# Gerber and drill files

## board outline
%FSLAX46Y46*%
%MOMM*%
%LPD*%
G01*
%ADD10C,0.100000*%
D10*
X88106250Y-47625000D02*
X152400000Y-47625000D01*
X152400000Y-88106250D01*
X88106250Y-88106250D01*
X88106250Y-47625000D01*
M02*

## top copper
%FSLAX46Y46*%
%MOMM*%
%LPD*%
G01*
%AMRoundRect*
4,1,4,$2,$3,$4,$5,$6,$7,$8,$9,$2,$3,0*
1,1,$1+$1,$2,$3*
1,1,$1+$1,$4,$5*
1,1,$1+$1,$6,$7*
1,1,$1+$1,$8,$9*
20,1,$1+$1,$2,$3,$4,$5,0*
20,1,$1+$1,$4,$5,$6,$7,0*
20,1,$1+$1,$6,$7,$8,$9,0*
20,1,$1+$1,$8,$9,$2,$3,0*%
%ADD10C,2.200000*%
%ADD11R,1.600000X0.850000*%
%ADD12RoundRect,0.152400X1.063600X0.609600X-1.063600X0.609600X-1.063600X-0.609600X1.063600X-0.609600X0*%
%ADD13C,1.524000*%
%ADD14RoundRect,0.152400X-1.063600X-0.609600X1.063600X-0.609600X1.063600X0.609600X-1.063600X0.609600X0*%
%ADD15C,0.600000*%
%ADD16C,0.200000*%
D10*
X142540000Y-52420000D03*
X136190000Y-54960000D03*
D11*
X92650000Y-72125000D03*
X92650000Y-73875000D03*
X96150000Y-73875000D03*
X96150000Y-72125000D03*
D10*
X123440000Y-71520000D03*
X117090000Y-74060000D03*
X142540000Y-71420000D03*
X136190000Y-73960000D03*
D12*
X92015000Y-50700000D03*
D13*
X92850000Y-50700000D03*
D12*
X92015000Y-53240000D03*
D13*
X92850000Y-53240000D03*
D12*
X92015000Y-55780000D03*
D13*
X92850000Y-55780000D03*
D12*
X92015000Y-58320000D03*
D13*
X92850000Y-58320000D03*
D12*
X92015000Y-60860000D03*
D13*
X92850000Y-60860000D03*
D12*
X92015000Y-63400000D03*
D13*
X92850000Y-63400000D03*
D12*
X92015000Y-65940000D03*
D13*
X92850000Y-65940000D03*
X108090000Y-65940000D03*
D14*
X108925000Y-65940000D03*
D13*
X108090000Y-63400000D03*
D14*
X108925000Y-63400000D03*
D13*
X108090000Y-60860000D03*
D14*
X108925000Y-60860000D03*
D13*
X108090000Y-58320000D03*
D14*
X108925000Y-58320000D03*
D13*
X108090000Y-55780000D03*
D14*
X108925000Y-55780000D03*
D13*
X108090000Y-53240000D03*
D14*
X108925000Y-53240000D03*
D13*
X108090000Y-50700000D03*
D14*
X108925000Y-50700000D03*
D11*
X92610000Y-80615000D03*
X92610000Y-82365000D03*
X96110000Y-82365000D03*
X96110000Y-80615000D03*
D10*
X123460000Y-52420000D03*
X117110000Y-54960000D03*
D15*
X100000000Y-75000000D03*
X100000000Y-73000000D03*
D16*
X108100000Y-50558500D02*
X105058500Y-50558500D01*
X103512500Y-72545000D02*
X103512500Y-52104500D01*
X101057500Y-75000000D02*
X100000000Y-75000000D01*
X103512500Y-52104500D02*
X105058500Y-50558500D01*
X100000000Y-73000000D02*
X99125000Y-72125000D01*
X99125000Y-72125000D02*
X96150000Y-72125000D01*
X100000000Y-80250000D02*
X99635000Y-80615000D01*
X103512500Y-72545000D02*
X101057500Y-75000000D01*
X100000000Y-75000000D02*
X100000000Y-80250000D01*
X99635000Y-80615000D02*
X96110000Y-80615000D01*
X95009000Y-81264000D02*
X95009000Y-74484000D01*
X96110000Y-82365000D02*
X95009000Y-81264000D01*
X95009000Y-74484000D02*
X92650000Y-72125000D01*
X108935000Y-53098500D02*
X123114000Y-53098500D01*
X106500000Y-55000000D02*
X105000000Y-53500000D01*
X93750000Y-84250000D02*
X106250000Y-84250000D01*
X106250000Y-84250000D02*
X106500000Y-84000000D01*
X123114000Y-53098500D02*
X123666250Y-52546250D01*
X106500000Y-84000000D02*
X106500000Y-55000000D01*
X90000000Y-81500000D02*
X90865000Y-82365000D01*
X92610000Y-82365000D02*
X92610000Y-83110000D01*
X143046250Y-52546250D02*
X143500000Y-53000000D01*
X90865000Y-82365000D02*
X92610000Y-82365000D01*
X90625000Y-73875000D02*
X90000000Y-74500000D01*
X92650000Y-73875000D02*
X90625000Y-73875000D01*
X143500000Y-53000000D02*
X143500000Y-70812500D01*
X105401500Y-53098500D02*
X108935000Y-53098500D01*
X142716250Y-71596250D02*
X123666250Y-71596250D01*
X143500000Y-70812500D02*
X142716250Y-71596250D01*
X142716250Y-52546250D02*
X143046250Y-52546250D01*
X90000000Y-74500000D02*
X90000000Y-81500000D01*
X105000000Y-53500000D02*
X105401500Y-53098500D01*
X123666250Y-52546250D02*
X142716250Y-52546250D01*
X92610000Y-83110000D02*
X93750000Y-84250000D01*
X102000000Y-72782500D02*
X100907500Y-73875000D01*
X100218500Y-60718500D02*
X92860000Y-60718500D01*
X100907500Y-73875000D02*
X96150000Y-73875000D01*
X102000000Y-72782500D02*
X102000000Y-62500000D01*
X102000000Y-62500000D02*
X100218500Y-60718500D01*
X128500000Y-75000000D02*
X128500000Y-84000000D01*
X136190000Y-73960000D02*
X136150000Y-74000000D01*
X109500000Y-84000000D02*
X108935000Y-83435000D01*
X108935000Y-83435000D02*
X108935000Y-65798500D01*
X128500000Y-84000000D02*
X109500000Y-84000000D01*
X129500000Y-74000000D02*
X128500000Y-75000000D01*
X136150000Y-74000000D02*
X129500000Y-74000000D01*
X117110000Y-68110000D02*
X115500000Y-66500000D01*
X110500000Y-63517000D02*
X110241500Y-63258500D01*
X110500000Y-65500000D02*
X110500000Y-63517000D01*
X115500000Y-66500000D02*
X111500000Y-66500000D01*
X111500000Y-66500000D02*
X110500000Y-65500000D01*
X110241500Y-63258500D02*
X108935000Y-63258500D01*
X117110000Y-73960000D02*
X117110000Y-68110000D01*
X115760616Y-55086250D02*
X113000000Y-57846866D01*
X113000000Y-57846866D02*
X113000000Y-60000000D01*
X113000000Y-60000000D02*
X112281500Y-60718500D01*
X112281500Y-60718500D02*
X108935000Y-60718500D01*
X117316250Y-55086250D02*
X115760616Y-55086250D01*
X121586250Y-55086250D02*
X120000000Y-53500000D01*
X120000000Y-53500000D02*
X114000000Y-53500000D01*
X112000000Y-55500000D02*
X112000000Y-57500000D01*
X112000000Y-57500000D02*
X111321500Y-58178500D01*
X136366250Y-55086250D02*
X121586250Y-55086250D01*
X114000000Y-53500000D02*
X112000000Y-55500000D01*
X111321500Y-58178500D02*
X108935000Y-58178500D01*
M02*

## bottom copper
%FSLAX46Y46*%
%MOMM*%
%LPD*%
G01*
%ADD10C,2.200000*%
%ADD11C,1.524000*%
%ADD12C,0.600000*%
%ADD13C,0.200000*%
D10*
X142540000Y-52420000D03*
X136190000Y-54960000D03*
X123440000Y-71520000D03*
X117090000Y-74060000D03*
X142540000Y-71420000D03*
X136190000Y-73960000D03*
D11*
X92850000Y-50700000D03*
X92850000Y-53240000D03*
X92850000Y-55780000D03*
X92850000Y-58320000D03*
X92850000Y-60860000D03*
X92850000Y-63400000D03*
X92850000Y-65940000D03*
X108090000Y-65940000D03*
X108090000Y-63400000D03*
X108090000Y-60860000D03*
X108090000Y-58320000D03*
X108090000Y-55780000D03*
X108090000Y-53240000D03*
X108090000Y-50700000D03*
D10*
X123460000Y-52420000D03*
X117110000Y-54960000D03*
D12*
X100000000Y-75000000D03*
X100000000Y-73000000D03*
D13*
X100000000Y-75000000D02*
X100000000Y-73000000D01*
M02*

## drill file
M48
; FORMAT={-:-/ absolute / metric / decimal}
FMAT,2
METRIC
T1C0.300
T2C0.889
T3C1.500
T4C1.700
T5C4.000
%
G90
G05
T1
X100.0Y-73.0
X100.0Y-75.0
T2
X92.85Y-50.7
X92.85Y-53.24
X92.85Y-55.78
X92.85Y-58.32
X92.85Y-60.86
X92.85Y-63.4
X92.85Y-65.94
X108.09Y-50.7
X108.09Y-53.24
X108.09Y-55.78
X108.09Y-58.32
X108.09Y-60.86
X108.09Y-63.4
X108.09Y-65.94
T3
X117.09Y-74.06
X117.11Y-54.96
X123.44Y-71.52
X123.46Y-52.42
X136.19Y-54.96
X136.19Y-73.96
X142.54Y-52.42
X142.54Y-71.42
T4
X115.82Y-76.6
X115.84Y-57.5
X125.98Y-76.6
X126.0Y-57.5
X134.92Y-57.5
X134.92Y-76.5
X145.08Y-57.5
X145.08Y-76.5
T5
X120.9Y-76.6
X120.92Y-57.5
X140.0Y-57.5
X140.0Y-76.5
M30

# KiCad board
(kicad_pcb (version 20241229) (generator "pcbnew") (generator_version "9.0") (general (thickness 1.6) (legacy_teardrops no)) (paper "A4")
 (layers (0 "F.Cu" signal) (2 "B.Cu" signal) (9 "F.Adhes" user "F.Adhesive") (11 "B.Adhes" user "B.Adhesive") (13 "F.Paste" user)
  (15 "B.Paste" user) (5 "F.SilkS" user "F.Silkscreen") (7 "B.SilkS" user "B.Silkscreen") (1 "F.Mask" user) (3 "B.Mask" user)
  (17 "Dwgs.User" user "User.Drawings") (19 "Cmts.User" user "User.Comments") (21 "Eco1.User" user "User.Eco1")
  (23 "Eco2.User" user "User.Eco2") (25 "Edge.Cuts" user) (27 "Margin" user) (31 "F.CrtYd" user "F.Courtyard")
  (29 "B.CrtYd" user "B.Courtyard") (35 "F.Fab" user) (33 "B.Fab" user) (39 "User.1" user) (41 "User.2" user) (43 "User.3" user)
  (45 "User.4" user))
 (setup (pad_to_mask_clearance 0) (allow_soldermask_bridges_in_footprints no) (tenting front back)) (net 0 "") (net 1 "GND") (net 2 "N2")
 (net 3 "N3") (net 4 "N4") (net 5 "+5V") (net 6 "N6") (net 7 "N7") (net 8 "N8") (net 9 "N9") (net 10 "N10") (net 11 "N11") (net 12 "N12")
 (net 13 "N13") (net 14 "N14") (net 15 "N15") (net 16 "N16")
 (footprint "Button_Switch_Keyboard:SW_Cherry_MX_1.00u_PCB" (layer "F.Cu") (at 142.54 52.42)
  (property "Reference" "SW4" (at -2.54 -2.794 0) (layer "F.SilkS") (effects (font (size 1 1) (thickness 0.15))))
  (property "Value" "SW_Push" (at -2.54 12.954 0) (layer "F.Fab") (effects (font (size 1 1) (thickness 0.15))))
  (pad "" np_thru_hole circle (at -7.62 5.08) (size 1.7 1.7) (drill 1.7) (layers "*.Cu" "*.Mask"))
  (pad "" np_thru_hole circle (at -2.54 5.08) (size 4 4) (drill 4) (layers "*.Cu" "*.Mask"))
  (pad "" np_thru_hole circle (at 2.54 5.08) (size 1.7 1.7) (drill 1.7) (layers "*.Cu" "*.Mask"))
  (pad "1" thru_hole circle (at 0 0) (size 2.2 2.2) (drill 1.5) (layers "*.Cu" "*.Mask") (remove_unused_layers no) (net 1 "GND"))
  (pad "2" thru_hole circle (at -6.35 2.54) (size 2.2 2.2) (drill 1.5) (layers "*.Cu" "*.Mask") (remove_unused_layers no) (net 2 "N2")))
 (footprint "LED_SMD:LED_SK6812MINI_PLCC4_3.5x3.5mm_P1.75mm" (layer "F.Cu") (at 94.4 73)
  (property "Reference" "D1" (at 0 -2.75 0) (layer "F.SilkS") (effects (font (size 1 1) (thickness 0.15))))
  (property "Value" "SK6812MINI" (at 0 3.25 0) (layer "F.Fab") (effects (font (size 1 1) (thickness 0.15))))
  (pad "1" smd rect (at -1.75 -0.875) (size 1.6 0.85) (layers "F.Cu" "F.Mask" "F.Paste") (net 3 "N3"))
  (pad "2" smd rect (at -1.75 0.875) (size 1.6 0.85) (layers "F.Cu" "F.Mask" "F.Paste") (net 1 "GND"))
  (pad "3" smd rect (at 1.75 0.875) (size 1.6 0.85) (layers "F.Cu" "F.Mask" "F.Paste") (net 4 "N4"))
  (pad "4" smd rect (at 1.75 -0.875) (size 1.6 0.85) (layers "F.Cu" "F.Mask" "F.Paste") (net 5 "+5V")))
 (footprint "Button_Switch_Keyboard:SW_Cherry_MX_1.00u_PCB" (layer "F.Cu") (at 123.44 71.52)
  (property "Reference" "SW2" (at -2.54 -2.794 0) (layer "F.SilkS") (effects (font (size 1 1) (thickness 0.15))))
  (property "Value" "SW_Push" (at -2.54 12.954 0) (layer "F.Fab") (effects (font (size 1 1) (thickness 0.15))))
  (pad "" np_thru_hole circle (at -7.62 5.08) (size 1.7 1.7) (drill 1.7) (layers "*.Cu" "*.Mask"))
  (pad "" np_thru_hole circle (at -2.54 5.08) (size 4 4) (drill 4) (layers "*.Cu" "*.Mask"))
  (pad "" np_thru_hole circle (at 2.54 5.08) (size 1.7 1.7) (drill 1.7) (layers "*.Cu" "*.Mask"))
  (pad "1" thru_hole circle (at 0 0) (size 2.2 2.2) (drill 1.5) (layers "*.Cu" "*.Mask") (remove_unused_layers no) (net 1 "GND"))
  (pad "2" thru_hole circle (at -6.35 2.54) (size 2.2 2.2) (drill 1.5) (layers "*.Cu" "*.Mask") (remove_unused_layers no) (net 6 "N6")))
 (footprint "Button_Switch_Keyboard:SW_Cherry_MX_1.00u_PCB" (layer "F.Cu") (at 142.54 71.42)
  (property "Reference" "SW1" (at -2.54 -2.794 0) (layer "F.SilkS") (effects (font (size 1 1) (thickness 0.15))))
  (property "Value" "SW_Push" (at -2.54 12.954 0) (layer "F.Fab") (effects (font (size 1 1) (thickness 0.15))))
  (pad "" np_thru_hole circle (at -7.62 5.08) (size 1.7 1.7) (drill 1.7) (layers "*.Cu" "*.Mask"))
  (pad "" np_thru_hole circle (at -2.54 5.08) (size 4 4) (drill 4) (layers "*.Cu" "*.Mask"))
  (pad "" np_thru_hole circle (at 2.54 5.08) (size 1.7 1.7) (drill 1.7) (layers "*.Cu" "*.Mask"))
  (pad "1" thru_hole circle (at 0 0) (size 2.2 2.2) (drill 1.5) (layers "*.Cu" "*.Mask") (remove_unused_layers no) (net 1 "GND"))
  (pad "2" thru_hole circle (at -6.35 2.54) (size 2.2 2.2) (drill 1.5) (layers "*.Cu" "*.Mask") (remove_unused_layers no) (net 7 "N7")))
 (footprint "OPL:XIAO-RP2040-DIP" (layer "F.Cu") (at 100.47 58.32)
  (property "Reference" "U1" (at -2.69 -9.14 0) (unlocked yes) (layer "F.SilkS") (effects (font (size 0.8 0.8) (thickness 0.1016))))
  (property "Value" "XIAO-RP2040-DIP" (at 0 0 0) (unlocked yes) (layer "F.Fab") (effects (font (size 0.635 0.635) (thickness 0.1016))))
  (pad "1" smd roundrect (at -8.455 -7.62 180) (size 2.432 1.524) (layers "F.Cu" "F.Mask") (roundrect_rratio 0.1) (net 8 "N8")
   (thermal_bridge_angle 45))
  (pad "1" thru_hole circle (at -7.62 -7.62 180) (size 1.524 1.524) (drill 0.889) (layers "*.Cu" "*.Mask") (remove_unused_layers no)
   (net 8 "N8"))
  (pad "2" smd roundrect (at -8.455 -5.08 180) (size 2.432 1.524) (layers "F.Cu" "F.Mask") (roundrect_rratio 0.1) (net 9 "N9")
   (thermal_bridge_angle 45))
  (pad "2" thru_hole circle (at -7.62 -5.08 180) (size 1.524 1.524) (drill 0.889) (layers "*.Cu" "*.Mask") (remove_unused_layers no)
   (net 9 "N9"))
  (pad "3" smd roundrect (at -8.455 -2.54 180) (size 2.432 1.524) (layers "F.Cu" "F.Mask") (roundrect_rratio 0.1) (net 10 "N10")
   (thermal_bridge_angle 45))
  (pad "3" thru_hole circle (at -7.62 -2.54 180) (size 1.524 1.524) (drill 0.889) (layers "*.Cu" "*.Mask") (remove_unused_layers no)
   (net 10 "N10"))
  (pad "4" smd roundrect (at -8.455 0 180) (size 2.432 1.524) (layers "F.Cu" "F.Mask") (roundrect_rratio 0.1) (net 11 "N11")
   (thermal_bridge_angle 45))
  (pad "4" thru_hole circle (at -7.62 0 180) (size 1.524 1.524) (drill 0.889) (layers "*.Cu" "*.Mask") (remove_unused_layers no)
   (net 11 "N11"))
  (pad "5" smd roundrect (at -8.455 2.54 180) (size 2.432 1.524) (layers "F.Cu" "F.Mask") (roundrect_rratio 0.1) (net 4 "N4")
   (thermal_bridge_angle 45))
  (pad "5" thru_hole circle (at -7.62 2.54 180) (size 1.524 1.524) (drill 0.889) (layers "*.Cu" "*.Mask") (remove_unused_layers no)
   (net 4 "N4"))
  (pad "6" smd roundrect (at -8.455 5.08 180) (size 2.432 1.524) (layers "F.Cu" "F.Mask") (roundrect_rratio 0.1) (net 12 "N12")
   (thermal_bridge_angle 45))
  (pad "6" thru_hole circle (at -7.62 5.08 180) (size 1.524 1.524) (drill 0.889) (layers "*.Cu" "*.Mask") (remove_unused_layers no)
   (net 12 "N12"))
  (pad "7" smd roundrect (at -8.455 7.62 180) (size 2.432 1.524) (layers "F.Cu" "F.Mask") (roundrect_rratio 0.1) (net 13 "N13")
   (thermal_bridge_angle 45))
  (pad "7" thru_hole circle (at -7.62 7.62 180) (size 1.524 1.524) (drill 0.889) (layers "*.Cu" "*.Mask") (remove_unused_layers no)
   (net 13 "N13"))
  (pad "8" thru_hole circle (at 7.62 7.62) (size 1.524 1.524) (drill 0.889) (layers "*.Cu" "*.Mask") (remove_unused_layers no) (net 7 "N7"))
  (pad "8" smd roundrect (at 8.455 7.62) (size 2.432 1.524) (layers "F.Cu" "F.Mask") (roundrect_rratio 0.1) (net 7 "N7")
   (thermal_bridge_angle 45))
  (pad "9" thru_hole circle (at 7.62 5.08) (size 1.524 1.524) (drill 0.889) (layers "*.Cu" "*.Mask") (remove_unused_layers no) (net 6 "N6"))
  (pad "9" smd roundrect (at 8.455 5.08) (size 2.432 1.524) (layers "F.Cu" "F.Mask") (roundrect_rratio 0.1) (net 6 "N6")
   (thermal_bridge_angle 45))
  (pad "10" thru_hole circle (at 7.62 2.54) (size 1.524 1.524) (drill 0.889) (layers "*.Cu" "*.Mask") (remove_unused_layers no)
   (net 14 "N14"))
  (pad "10" smd roundrect (at 8.455 2.54) (size 2.432 1.524) (layers "F.Cu" "F.Mask") (roundrect_rratio 0.1) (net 14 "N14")
   (thermal_bridge_angle 45))
  (pad "11" thru_hole circle (at 7.62 0) (size 1.524 1.524) (drill 0.889) (layers "*.Cu" "*.Mask") (remove_unused_layers no) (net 2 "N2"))
  (pad "11" smd roundrect (at 8.455 0) (size 2.432 1.524) (layers "F.Cu" "F.Mask") (roundrect_rratio 0.1) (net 2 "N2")
   (thermal_bridge_angle 45))
  (pad "12" thru_hole circle (at 7.62 -2.54) (size 1.524 1.524) (drill 0.889) (layers "*.Cu" "*.Mask") (remove_unused_layers no)
   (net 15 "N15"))
  (pad "12" smd roundrect (at 8.455 -2.54) (size 2.432 1.524) (layers "F.Cu" "F.Mask") (roundrect_rratio 0.1) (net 15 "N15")
   (thermal_bridge_angle 45))
  (pad "13" thru_hole circle (at 7.62 -5.08) (size 1.524 1.524) (drill 0.889) (layers "*.Cu" "*.Mask") (remove_unused_layers no)
   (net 1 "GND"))
  (pad "13" smd roundrect (at 8.455 -5.08) (size 2.432 1.524) (layers "F.Cu" "F.Mask") (roundrect_rratio 0.1) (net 1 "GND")
   (thermal_bridge_angle 45))
  (pad "14" thru_hole circle (at 7.62 -7.62) (size 1.524 1.524) (drill 0.889) (layers "*.Cu" "*.Mask") (remove_unused_layers no)
   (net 5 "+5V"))
  (pad "14" smd roundrect (at 8.455 -7.62) (size 2.432 1.524) (layers "F.Cu" "F.Mask") (roundrect_rratio 0.1) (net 5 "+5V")
   (thermal_bridge_angle 45)))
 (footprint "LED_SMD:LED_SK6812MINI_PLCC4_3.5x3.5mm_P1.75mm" (layer "F.Cu") (at 94.36 81.49)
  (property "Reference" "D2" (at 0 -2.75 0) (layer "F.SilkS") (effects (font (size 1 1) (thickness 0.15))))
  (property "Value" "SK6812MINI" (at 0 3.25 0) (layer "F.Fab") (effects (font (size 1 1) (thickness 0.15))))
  (pad "1" smd rect (at -1.75 -0.875) (size 1.6 0.85) (layers "F.Cu" "F.Mask" "F.Paste") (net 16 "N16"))
  (pad "2" smd rect (at -1.75 0.875) (size 1.6 0.85) (layers "F.Cu" "F.Mask" "F.Paste") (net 1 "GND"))
  (pad "3" smd rect (at 1.75 0.875) (size 1.6 0.85) (layers "F.Cu" "F.Mask" "F.Paste") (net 3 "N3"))
  (pad "4" smd rect (at 1.75 -0.875) (size 1.6 0.85) (layers "F.Cu" "F.Mask" "F.Paste") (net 5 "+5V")))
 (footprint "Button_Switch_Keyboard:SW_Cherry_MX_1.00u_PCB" (layer "F.Cu") (at 123.46 52.42)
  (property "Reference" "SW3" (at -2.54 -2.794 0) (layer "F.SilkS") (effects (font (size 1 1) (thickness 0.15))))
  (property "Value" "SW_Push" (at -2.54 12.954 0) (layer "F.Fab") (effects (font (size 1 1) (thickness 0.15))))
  (pad "" np_thru_hole circle (at -7.62 5.08) (size 1.7 1.7) (drill 1.7) (layers "*.Cu" "*.Mask"))
  (pad "" np_thru_hole circle (at -2.54 5.08) (size 4 4) (drill 4) (layers "*.Cu" "*.Mask"))
  (pad "" np_thru_hole circle (at 2.54 5.08) (size 1.7 1.7) (drill 1.7) (layers "*.Cu" "*.Mask"))
  (pad "1" thru_hole circle (at 0 0) (size 2.2 2.2) (drill 1.5) (layers "*.Cu" "*.Mask") (remove_unused_layers no) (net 1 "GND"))
  (pad "2" thru_hole circle (at -6.35 2.54) (size 2.2 2.2) (drill 1.5) (layers "*.Cu" "*.Mask") (remove_unused_layers no) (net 14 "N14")))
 (gr_rect (start 88.10625 47.625) (end 152.4 88.10625) (stroke (width 0.1) (type solid)) (fill no) (layer "Edge.Cuts"))
 (segment (start 108.1 50.5585) (end 105.0585 50.5585) (width 0.2) (layer "F.Cu") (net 5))
 (segment (start 103.5125 72.545) (end 103.5125 52.1045) (width 0.2) (layer "F.Cu") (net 5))
 (segment (start 101.0575 75) (end 100 75) (width 0.2) (layer "F.Cu") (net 5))
 (segment (start 103.5125 52.1045) (end 105.0585 50.5585) (width 0.2) (layer "F.Cu") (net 5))
 (segment (start 100 73) (end 99.125 72.125) (width 0.2) (layer "F.Cu") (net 5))
 (segment (start 99.125 72.125) (end 96.15 72.125) (width 0.2) (layer "F.Cu") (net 5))
 (segment (start 100 80.25) (end 99.635 80.615) (width 0.2) (layer "F.Cu") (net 5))
 (segment (start 103.5125 72.545) (end 101.0575 75) (width 0.2) (layer "F.Cu") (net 5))
 (segment (start 100 75) (end 100 80.25) (width 0.2) (layer "F.Cu") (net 5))
 (segment (start 99.635 80.615) (end 96.11 80.615) (width 0.2) (layer "F.Cu") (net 5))
 (via (at 100 75) (size 0.6) (drill 0.3) (layers "F.Cu" "B.Cu") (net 5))
 (via (at 100 73) (size 0.6) (drill 0.3) (layers "F.Cu" "B.Cu") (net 5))
 (segment (start 100 75) (end 100 73) (width 0.2) (layer "B.Cu") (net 5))
 (segment (start 95.009 81.264) (end 95.009 74.484) (width 0.2) (layer "F.Cu") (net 3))
 (segment (start 96.11 82.365) (end 95.009 81.264) (width 0.2) (layer "F.Cu") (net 3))
 (segment (start 95.009 74.484) (end 92.65 72.125) (width 0.2) (layer "F.Cu") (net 3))
 (segment (start 108.935 53.0985) (end 123.114 53.0985) (width 0.2) (layer "F.Cu") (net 1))
 (segment (start 106.5 55) (end 105 53.5) (width 0.2) (layer "F.Cu") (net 1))
 (segment (start 93.75 84.25) (end 106.25 84.25) (width 0.2) (layer "F.Cu") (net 1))
 (segment (start 106.25 84.25) (end 106.5 84) (width 0.2) (layer "F.Cu") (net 1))
 (segment (start 123.114 53.0985) (end 123.66625 52.54625) (width 0.2) (layer "F.Cu") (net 1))
 (segment (start 106.5 84) (end 106.5 55) (width 0.2) (layer "F.Cu") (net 1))
 (segment (start 90 81.5) (end 90.865 82.365) (width 0.2) (layer "F.Cu") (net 1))
 (segment (start 92.61 82.365) (end 92.61 83.11) (width 0.2) (layer "F.Cu") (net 1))
 (segment (start 143.04625 52.54625) (end 143.5 53) (width 0.2) (layer "F.Cu") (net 1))
 (segment (start 90.865 82.365) (end 92.61 82.365) (width 0.2) (layer "F.Cu") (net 1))
 (segment (start 90.625 73.875) (end 90 74.5) (width 0.2) (layer "F.Cu") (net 1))
 (segment (start 92.65 73.875) (end 90.625 73.875) (width 0.2) (layer "F.Cu") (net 1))
 (segment (start 143.5 53) (end 143.5 70.8125) (width 0.2) (layer "F.Cu") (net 1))
 (segment (start 105.4015 53.0985) (end 108.935 53.0985) (width 0.2) (layer "F.Cu") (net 1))
 (segment (start 142.71625 71.59625) (end 123.66625 71.59625) (width 0.2) (layer "F.Cu") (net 1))
 (segment (start 143.5 70.8125) (end 142.71625 71.59625) (width 0.2) (layer "F.Cu") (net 1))
 (segment (start 142.71625 52.54625) (end 143.04625 52.54625) (width 0.2) (layer "F.Cu") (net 1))
 (segment (start 90 74.5) (end 90 81.5) (width 0.2) (layer "F.Cu") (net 1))
 (segment (start 105 53.5) (end 105.4015 53.0985) (width 0.2) (layer "F.Cu") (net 1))
 (segment (start 123.66625 52.54625) (end 142.71625 52.54625) (width 0.2) (layer "F.Cu") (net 1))
 (segment (start 92.61 83.11) (end 93.75 84.25) (width 0.2) (layer "F.Cu") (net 1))
 (segment (start 102 72.7825) (end 100.9075 73.875) (width 0.2) (layer "F.Cu") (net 4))
 (segment (start 100.2185 60.7185) (end 92.86 60.7185) (width 0.2) (layer "F.Cu") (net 4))
 (segment (start 100.9075 73.875) (end 96.15 73.875) (width 0.2) (layer "F.Cu") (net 4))
 (segment (start 102 72.7825) (end 102 62.5) (width 0.2) (layer "F.Cu") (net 4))
 (segment (start 102 62.5) (end 100.2185 60.7185) (width 0.2) (layer "F.Cu") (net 4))
 (segment (start 128.5 75) (end 128.5 84) (width 0.2) (layer "F.Cu") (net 7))
 (segment (start 136.19 73.96) (end 136.15 74) (width 0.2) (layer "F.Cu") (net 7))
 (segment (start 109.5 84) (end 108.935 83.435) (width 0.2) (layer "F.Cu") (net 7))
 (segment (start 108.935 83.435) (end 108.935 65.7985) (width 0.2) (layer "F.Cu") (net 7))
 (segment (start 128.5 84) (end 109.5 84) (width 0.2) (layer "F.Cu") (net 7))
 (segment (start 129.5 74) (end 128.5 75) (width 0.2) (layer "F.Cu") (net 7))
 (segment (start 136.15 74) (end 129.5 74) (width 0.2) (layer "F.Cu") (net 7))
 (segment (start 117.11 68.11) (end 115.5 66.5) (width 0.2) (layer "F.Cu") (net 6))
 (segment (start 110.5 63.517) (end 110.2415 63.2585) (width 0.2) (layer "F.Cu") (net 6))
 (segment (start 110.5 65.5) (end 110.5 63.517) (width 0.2) (layer "F.Cu") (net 6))
 (segment (start 115.5 66.5) (end 111.5 66.5) (width 0.2) (layer "F.Cu") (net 6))
 (segment (start 111.5 66.5) (end 110.5 65.5) (width 0.2) (layer "F.Cu") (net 6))
 (segment (start 110.2415 63.2585) (end 108.935 63.2585) (width 0.2) (layer "F.Cu") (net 6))
 (segment (start 117.11 73.96) (end 117.11 68.11) (width 0.2) (layer "F.Cu") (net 6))
 (segment (start 115.760616 55.08625) (end 113 57.846866) (width 0.2) (layer "F.Cu") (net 14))
 (segment (start 113 57.846866) (end 113 60) (width 0.2) (layer "F.Cu") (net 14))
 (segment (start 113 60) (end 112.2815 60.7185) (width 0.2) (layer "F.Cu") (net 14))
 (segment (start 112.2815 60.7185) (end 108.935 60.7185) (width 0.2) (layer "F.Cu") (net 14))
 (segment (start 117.31625 55.08625) (end 115.760616 55.08625) (width 0.2) (layer "F.Cu") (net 14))
 (segment (start 121.58625 55.08625) (end 120 53.5) (width 0.2) (layer "F.Cu") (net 2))
 (segment (start 120 53.5) (end 114 53.5) (width 0.2) (layer "F.Cu") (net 2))
 (segment (start 112 55.5) (end 112 57.5) (width 0.2) (layer "F.Cu") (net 2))
 (segment (start 112 57.5) (end 111.3215 58.1785) (width 0.2) (layer "F.Cu") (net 2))
 (segment (start 136.36625 55.08625) (end 121.58625 55.08625) (width 0.2) (layer "F.Cu") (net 2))
 (segment (start 114 53.5) (end 112 55.5) (width 0.2) (layer "F.Cu") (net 2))
 (segment (start 111.3215 58.1785) (end 108.935 58.1785) (width 0.2) (layer "F.Cu") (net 2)))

